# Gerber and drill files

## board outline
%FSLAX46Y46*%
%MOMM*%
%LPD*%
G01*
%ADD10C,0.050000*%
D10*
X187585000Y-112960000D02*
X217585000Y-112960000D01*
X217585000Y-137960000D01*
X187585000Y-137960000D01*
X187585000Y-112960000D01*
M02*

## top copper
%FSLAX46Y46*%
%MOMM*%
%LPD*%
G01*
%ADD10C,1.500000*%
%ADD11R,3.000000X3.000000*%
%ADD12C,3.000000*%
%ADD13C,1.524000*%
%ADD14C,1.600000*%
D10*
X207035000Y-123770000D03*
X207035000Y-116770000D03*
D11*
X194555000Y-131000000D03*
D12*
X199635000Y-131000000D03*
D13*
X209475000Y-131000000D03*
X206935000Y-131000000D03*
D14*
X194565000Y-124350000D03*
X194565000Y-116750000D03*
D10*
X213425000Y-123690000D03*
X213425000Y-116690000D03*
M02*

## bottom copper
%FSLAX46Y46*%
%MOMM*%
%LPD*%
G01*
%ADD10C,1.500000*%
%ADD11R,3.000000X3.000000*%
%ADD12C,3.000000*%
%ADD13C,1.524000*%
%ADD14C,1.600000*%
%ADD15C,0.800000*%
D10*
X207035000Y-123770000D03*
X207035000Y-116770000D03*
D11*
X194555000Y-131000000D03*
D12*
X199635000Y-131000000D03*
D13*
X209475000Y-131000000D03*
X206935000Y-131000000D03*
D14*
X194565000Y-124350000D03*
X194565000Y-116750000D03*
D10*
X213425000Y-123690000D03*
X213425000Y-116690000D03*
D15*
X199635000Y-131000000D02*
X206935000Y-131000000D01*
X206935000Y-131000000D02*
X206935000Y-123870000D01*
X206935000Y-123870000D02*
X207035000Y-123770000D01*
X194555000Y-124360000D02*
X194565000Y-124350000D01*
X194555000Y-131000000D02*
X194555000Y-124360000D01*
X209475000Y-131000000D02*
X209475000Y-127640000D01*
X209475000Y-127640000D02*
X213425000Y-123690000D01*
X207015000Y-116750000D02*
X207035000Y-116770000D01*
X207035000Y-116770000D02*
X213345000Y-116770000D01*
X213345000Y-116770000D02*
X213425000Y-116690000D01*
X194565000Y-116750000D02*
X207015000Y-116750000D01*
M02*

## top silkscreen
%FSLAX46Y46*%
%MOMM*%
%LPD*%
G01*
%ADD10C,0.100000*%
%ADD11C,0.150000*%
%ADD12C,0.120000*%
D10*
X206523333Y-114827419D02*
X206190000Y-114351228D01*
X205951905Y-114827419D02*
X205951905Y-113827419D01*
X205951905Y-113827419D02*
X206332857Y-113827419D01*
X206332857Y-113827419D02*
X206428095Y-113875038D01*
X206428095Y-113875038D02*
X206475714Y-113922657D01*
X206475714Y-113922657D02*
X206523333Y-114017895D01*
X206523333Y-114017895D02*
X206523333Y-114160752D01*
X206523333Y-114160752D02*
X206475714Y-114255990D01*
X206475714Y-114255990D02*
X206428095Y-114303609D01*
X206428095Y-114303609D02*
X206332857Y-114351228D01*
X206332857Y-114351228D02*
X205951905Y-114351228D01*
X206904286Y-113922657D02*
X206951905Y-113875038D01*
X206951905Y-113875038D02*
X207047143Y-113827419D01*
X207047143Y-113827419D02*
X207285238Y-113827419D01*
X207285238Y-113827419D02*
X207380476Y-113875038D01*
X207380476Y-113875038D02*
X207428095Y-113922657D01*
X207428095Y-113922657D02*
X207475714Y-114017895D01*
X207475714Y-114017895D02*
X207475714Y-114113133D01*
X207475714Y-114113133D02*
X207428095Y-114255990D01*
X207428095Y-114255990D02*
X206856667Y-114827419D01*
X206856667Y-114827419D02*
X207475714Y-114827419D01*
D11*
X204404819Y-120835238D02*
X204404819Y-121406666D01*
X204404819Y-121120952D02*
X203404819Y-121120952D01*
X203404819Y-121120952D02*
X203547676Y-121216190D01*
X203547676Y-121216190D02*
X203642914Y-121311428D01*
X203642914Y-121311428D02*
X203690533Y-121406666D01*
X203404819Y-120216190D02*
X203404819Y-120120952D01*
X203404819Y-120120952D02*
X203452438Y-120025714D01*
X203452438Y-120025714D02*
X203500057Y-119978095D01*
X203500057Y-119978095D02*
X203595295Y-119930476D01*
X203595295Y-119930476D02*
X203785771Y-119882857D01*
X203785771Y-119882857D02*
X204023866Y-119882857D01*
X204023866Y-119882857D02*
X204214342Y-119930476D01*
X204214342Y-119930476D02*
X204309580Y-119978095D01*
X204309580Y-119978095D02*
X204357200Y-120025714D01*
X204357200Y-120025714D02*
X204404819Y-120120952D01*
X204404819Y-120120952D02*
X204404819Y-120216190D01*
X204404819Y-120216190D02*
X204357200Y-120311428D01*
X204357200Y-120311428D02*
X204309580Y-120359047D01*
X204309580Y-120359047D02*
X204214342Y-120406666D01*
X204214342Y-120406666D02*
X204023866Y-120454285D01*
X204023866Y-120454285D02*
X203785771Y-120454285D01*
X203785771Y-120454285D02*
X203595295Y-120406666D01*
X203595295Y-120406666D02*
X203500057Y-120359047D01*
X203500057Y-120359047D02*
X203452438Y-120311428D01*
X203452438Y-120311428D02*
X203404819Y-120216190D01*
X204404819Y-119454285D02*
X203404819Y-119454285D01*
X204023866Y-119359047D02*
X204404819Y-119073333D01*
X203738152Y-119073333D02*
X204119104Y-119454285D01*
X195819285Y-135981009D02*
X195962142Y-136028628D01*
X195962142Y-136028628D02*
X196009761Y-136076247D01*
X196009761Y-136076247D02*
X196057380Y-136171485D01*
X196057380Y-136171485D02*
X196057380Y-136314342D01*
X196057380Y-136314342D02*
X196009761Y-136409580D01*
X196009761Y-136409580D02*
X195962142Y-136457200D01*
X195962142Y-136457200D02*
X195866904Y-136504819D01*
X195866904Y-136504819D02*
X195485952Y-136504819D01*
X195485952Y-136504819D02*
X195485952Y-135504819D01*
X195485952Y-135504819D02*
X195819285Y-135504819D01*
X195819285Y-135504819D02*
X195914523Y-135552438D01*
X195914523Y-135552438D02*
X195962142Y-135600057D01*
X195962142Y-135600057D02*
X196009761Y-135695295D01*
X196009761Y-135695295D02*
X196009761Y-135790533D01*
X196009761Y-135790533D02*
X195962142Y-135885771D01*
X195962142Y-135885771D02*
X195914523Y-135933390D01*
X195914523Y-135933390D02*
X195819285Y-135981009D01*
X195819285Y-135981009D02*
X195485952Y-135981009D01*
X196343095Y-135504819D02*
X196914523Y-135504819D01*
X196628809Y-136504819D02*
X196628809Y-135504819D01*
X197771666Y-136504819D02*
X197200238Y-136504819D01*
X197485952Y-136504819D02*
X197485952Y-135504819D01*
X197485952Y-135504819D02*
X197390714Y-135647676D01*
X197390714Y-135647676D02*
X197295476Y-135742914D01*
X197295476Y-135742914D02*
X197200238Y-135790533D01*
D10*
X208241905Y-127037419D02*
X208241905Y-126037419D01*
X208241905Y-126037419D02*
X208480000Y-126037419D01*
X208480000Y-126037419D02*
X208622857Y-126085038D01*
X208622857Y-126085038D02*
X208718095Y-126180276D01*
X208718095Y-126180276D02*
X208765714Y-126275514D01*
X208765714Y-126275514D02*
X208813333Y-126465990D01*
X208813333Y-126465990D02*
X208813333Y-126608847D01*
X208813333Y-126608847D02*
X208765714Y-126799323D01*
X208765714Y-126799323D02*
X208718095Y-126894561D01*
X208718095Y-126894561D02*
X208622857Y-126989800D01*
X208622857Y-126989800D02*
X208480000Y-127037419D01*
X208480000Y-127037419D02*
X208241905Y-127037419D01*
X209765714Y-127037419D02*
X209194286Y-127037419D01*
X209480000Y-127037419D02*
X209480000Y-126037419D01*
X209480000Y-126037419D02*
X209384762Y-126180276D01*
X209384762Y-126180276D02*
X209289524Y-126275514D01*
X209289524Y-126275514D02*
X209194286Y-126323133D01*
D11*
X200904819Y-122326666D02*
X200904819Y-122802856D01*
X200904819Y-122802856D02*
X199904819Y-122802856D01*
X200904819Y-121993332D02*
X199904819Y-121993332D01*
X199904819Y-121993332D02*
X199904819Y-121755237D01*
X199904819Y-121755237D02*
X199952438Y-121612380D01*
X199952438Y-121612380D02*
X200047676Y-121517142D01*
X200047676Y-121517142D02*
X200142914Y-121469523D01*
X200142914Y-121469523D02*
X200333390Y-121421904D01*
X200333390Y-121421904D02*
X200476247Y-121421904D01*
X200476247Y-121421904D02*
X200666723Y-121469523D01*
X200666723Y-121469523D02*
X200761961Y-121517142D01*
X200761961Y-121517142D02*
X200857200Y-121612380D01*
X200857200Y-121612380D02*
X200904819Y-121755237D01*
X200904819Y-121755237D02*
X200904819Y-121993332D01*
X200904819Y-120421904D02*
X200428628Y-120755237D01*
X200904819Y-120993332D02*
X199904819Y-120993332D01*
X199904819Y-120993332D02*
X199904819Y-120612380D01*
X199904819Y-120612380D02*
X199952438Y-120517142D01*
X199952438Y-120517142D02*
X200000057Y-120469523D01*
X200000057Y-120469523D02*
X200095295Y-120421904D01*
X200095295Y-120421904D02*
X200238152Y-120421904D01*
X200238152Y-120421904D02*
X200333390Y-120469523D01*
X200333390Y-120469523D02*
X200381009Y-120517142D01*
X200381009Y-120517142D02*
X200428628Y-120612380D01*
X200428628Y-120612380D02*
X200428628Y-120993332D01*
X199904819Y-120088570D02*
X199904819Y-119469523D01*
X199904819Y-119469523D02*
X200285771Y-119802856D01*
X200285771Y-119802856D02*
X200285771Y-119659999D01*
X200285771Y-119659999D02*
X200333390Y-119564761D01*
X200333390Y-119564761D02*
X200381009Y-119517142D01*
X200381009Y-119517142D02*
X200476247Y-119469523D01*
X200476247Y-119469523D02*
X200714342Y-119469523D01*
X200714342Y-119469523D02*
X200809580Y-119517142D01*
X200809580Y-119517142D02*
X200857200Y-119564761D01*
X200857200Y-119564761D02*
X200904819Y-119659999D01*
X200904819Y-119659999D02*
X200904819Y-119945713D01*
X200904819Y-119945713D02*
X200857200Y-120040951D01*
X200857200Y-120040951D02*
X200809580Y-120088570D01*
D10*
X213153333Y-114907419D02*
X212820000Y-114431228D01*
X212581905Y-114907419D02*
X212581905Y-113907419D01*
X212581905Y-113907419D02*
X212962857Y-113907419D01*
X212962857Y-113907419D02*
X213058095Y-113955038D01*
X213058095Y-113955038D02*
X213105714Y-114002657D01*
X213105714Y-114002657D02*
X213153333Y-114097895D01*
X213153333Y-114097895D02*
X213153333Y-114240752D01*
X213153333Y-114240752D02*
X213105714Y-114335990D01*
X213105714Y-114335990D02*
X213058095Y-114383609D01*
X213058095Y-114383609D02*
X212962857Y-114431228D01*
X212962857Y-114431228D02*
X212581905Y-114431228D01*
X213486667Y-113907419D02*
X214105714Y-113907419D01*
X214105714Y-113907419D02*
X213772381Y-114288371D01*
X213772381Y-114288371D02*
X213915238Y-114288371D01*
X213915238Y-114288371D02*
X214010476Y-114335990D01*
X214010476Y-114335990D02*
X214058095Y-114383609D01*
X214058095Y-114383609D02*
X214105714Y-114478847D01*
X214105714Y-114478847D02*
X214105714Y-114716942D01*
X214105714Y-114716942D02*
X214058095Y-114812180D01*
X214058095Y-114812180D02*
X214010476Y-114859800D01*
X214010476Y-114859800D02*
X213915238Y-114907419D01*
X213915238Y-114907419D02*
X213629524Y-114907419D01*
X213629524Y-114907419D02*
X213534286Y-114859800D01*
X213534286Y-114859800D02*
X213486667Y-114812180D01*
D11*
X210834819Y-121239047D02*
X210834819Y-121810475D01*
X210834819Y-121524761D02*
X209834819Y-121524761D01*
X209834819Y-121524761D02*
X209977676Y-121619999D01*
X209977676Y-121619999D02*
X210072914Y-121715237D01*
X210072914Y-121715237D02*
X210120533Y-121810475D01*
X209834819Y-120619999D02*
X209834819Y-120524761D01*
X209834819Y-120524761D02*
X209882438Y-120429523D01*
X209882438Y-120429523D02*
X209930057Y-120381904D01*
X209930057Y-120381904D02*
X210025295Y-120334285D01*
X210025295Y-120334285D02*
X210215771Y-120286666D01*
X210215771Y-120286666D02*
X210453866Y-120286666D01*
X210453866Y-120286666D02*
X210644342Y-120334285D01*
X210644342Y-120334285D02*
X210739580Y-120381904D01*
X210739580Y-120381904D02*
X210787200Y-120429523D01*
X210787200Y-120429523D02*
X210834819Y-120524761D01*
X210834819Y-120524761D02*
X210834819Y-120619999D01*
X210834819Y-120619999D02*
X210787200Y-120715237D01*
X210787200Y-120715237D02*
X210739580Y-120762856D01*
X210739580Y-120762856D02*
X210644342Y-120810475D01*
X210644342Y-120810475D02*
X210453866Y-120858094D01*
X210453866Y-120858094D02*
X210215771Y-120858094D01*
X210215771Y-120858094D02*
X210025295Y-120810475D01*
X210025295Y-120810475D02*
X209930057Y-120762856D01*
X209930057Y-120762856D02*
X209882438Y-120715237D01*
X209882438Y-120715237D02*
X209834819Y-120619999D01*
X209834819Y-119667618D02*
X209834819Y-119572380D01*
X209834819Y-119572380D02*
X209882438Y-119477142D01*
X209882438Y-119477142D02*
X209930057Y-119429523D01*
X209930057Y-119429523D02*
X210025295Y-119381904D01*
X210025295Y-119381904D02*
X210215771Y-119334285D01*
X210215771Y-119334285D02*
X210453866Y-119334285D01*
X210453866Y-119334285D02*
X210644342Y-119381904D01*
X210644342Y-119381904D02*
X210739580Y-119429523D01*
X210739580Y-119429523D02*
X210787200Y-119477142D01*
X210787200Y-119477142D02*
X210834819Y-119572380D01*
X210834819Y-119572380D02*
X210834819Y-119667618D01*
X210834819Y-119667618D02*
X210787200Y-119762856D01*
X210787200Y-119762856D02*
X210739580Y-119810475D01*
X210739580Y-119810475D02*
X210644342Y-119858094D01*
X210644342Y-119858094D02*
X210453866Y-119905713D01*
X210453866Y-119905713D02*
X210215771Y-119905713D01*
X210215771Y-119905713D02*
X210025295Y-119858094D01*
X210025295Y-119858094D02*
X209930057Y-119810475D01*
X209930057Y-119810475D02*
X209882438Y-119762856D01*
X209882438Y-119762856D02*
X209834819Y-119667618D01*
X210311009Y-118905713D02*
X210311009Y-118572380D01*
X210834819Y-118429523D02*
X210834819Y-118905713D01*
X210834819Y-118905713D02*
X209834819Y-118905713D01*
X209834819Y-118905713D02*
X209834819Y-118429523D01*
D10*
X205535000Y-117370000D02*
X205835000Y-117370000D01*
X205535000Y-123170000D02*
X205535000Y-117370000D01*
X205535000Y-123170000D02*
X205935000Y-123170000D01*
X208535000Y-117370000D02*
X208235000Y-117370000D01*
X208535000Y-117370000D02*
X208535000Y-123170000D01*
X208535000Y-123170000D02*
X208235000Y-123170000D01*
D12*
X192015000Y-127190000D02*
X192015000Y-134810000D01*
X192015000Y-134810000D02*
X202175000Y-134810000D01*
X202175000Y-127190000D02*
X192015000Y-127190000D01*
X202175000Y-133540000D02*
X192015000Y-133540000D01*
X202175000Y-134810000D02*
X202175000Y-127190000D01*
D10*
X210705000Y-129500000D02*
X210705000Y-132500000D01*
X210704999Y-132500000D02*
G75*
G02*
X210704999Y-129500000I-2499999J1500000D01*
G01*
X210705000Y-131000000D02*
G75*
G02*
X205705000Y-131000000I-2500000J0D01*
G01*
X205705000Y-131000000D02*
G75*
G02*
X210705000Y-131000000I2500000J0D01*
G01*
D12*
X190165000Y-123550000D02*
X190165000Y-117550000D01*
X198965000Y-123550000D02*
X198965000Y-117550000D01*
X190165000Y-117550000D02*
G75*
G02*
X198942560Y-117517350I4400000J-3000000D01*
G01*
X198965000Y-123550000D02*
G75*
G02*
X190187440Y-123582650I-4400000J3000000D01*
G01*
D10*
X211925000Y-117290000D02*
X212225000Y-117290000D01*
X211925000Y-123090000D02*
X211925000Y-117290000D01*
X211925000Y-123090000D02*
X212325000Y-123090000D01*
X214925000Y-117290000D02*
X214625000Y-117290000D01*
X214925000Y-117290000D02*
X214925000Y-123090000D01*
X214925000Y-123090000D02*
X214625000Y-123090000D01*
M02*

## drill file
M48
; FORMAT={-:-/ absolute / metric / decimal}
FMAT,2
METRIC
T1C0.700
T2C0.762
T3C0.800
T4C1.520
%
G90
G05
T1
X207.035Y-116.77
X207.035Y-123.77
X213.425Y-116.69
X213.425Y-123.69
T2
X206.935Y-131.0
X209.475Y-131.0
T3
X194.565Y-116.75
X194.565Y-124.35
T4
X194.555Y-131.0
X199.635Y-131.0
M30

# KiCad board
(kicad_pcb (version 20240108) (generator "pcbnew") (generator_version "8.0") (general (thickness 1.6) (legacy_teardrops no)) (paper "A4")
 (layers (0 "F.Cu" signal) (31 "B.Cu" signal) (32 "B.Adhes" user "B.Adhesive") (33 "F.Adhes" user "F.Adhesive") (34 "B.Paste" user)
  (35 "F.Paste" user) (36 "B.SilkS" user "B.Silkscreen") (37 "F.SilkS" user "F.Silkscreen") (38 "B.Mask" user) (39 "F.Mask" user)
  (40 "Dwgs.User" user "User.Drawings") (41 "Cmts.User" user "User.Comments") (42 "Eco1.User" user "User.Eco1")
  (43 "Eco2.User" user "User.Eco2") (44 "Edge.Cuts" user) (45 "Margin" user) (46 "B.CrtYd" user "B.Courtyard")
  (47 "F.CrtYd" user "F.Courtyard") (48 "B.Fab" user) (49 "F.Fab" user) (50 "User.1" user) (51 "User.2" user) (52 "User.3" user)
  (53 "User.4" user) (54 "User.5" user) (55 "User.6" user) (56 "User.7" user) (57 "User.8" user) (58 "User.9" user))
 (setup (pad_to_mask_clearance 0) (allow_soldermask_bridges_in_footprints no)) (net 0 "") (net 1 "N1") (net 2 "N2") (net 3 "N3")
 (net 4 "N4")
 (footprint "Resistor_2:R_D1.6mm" (layer "F.Cu") (at 207.035 120.27 90)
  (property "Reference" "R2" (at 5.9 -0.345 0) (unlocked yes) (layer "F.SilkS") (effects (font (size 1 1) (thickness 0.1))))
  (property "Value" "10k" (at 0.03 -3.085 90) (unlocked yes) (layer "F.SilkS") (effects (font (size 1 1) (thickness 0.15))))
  (fp_line (start 2.9 -1.5) (end 2.9 -1.2) (stroke (width 0.1) (type default)) (layer "F.SilkS"))
  (fp_line (start -2.9 -1.5) (end 2.9 -1.5) (stroke (width 0.1) (type default)) (layer "F.SilkS"))
  (fp_line (start -2.9 -1.5) (end -2.9 -1.1) (stroke (width 0.1) (type default)) (layer "F.SilkS"))
  (fp_line (start 2.9 1.5) (end 2.9 1.2) (stroke (width 0.1) (type default)) (layer "F.SilkS"))
  (fp_line (start 2.9 1.5) (end -2.9 1.5) (stroke (width 0.1) (type default)) (layer "F.SilkS"))
  (fp_line (start -2.9 1.5) (end -2.9 1.2) (stroke (width 0.1) (type default)) (layer "F.SilkS"))
  (pad "1" thru_hole circle (at -3.5 0 90) (size 1.5 1.5) (drill 0.7) (layers "*.Cu" "*.Mask") (remove_unused_layers no) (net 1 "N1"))
  (pad "2" thru_hole circle (at 3.5 0 90) (size 1.5 1.5) (drill 0.7) (layers "*.Cu" "*.Mask") (remove_unused_layers no) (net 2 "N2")))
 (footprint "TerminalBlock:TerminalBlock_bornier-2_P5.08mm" (layer "F.Cu") (at 194.555 131)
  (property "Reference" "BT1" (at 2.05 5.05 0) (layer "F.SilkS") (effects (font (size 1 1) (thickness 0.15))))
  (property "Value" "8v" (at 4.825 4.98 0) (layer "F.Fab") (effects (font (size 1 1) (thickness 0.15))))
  (fp_line (start -2.54 -3.81) (end -2.54 3.81) (stroke (width 0.12) (type solid)) (layer "F.SilkS"))
  (fp_line (start -2.54 3.81) (end 7.62 3.81) (stroke (width 0.12) (type solid)) (layer "F.SilkS"))
  (fp_line (start 7.62 -3.81) (end -2.54 -3.81) (stroke (width 0.12) (type solid)) (layer "F.SilkS"))
  (fp_line (start 7.62 2.54) (end -2.54 2.54) (stroke (width 0.12) (type solid)) (layer "F.SilkS"))
  (fp_line (start 7.62 3.81) (end 7.62 -3.81) (stroke (width 0.12) (type solid)) (layer "F.SilkS"))
  (pad "1" thru_hole rect (at 0 0) (size 3 3) (drill 1.52) (layers "*.Cu" "*.Mask") (remove_unused_layers no) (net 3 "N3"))
  (pad "2" thru_hole circle (at 5.08 0) (size 3 3) (drill 1.52) (layers "*.Cu" "*.Mask") (remove_unused_layers no) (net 1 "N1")))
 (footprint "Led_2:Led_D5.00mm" (layer "F.Cu") (at 208.205 131 180)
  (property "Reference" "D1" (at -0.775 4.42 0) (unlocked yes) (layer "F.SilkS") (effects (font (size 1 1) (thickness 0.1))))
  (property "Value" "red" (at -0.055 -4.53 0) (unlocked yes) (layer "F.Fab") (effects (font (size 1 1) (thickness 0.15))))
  (fp_line (start -2.5 1.5) (end -2.5 -1.5) (stroke (width 0.1) (type default)) (layer "F.SilkS"))
  (fp_arc (start -2.499999 -1.5) (mid 2.915475 0) (end -2.499999 1.5) (stroke (width 0.1) (type default)) (layer "F.SilkS"))
  (fp_circle (center 0 0) (end -2.5 0) (stroke (width 0.1) (type default)) (fill none) (layer "F.SilkS"))
  (pad "1" thru_hole circle (at -1.27 0 180) (size 1.524 1.524) (drill 0.762) (layers "*.Cu" "*.Mask") (remove_unused_layers no)
   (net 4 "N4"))
  (pad "2" thru_hole circle (at 1.27 0 180) (size 1.524 1.524) (drill 0.762) (layers "*.Cu" "*.Mask") (remove_unused_layers no) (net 1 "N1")))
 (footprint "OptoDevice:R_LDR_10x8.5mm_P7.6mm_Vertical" (layer "F.Cu") (at 194.565 124.35 90)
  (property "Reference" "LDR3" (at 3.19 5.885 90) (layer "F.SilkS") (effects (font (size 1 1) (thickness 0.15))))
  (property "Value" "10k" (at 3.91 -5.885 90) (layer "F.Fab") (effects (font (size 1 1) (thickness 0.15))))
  (fp_line (start 0.8 -4.4) (end 6.8 -4.4) (stroke (width 0.12) (type solid)) (layer "F.SilkS"))
  (fp_line (start 0.8 4.4) (end 6.8 4.4) (stroke (width 0.12) (type solid)) (layer "F.SilkS"))
  (fp_arc (start 6.8 -4.4) (mid 9.125374 -0.019809) (end 6.83265 4.37756) (stroke (width 0.12) (type solid)) (layer "F.SilkS"))
  (fp_arc (start 0.8 4.4) (mid -1.525374 0.019809) (end 0.76735 -4.37756) (stroke (width 0.12) (type solid)) (layer "F.SilkS"))
  (pad "1" thru_hole circle (at 0 0 90) (size 1.6 1.6) (drill 0.8) (layers "*.Cu" "*.Mask") (remove_unused_layers no) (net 3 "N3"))
  (pad "2" thru_hole circle (at 7.6 0 90) (size 1.6 1.6) (drill 0.8) (layers "*.Cu" "*.Mask") (remove_unused_layers no) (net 2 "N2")))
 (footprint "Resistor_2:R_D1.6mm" (layer "F.Cu") (at 213.425 120.19 90)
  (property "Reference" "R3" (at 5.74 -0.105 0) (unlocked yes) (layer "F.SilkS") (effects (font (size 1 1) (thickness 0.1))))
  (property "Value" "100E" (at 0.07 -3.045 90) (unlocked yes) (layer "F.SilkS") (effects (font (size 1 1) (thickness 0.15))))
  (fp_line (start 2.9 -1.5) (end 2.9 -1.2) (stroke (width 0.1) (type default)) (layer "F.SilkS"))
  (fp_line (start -2.9 -1.5) (end 2.9 -1.5) (stroke (width 0.1) (type default)) (layer "F.SilkS"))
  (fp_line (start -2.9 -1.5) (end -2.9 -1.1) (stroke (width 0.1) (type default)) (layer "F.SilkS"))
  (fp_line (start 2.9 1.5) (end 2.9 1.2) (stroke (width 0.1) (type default)) (layer "F.SilkS"))
  (fp_line (start 2.9 1.5) (end -2.9 1.5) (stroke (width 0.1) (type default)) (layer "F.SilkS"))
  (fp_line (start -2.9 1.5) (end -2.9 1.2) (stroke (width 0.1) (type default)) (layer "F.SilkS"))
  (pad "1" thru_hole circle (at -3.5 0 90) (size 1.5 1.5) (drill 0.7) (layers "*.Cu" "*.Mask") (remove_unused_layers no) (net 4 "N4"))
  (pad "2" thru_hole circle (at 3.5 0 90) (size 1.5 1.5) (drill 0.7) (layers "*.Cu" "*.Mask") (remove_unused_layers no) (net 2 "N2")))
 (gr_rect (start 187.585 112.96) (end 217.585 137.96) (stroke (width 0.05) (type default)) (fill none) (layer "Edge.Cuts"))
 (segment (start 199.635 131) (end 206.935 131) (width 0.8) (layer "B.Cu") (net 1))
 (segment (start 206.935 131) (end 206.935 123.87) (width 0.8) (layer "B.Cu") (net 1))
 (segment (start 206.935 123.87) (end 207.035 123.77) (width 0.8) (layer "B.Cu") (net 1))
 (segment (start 194.555 124.36) (end 194.565 124.35) (width 0.8) (layer "B.Cu") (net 3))
 (segment (start 194.555 131) (end 194.555 124.36) (width 0.8) (layer "B.Cu") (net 3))
 (segment (start 209.475 131) (end 209.475 127.64) (width 0.8) (layer "B.Cu") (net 4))
 (segment (start 209.475 127.64) (end 213.425 123.69) (width 0.8) (layer "B.Cu") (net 4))
 (segment (start 207.015 116.75) (end 207.035 116.77) (width 0.8) (layer "B.Cu") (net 2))
 (segment (start 207.035 116.77) (end 213.345 116.77) (width 0.8) (layer "B.Cu") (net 2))
 (segment (start 213.345 116.77) (end 213.425 116.69) (width 0.8) (layer "B.Cu") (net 2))
 (segment (start 194.565 116.75) (end 207.015 116.75) (width 0.8) (layer "B.Cu") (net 2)))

